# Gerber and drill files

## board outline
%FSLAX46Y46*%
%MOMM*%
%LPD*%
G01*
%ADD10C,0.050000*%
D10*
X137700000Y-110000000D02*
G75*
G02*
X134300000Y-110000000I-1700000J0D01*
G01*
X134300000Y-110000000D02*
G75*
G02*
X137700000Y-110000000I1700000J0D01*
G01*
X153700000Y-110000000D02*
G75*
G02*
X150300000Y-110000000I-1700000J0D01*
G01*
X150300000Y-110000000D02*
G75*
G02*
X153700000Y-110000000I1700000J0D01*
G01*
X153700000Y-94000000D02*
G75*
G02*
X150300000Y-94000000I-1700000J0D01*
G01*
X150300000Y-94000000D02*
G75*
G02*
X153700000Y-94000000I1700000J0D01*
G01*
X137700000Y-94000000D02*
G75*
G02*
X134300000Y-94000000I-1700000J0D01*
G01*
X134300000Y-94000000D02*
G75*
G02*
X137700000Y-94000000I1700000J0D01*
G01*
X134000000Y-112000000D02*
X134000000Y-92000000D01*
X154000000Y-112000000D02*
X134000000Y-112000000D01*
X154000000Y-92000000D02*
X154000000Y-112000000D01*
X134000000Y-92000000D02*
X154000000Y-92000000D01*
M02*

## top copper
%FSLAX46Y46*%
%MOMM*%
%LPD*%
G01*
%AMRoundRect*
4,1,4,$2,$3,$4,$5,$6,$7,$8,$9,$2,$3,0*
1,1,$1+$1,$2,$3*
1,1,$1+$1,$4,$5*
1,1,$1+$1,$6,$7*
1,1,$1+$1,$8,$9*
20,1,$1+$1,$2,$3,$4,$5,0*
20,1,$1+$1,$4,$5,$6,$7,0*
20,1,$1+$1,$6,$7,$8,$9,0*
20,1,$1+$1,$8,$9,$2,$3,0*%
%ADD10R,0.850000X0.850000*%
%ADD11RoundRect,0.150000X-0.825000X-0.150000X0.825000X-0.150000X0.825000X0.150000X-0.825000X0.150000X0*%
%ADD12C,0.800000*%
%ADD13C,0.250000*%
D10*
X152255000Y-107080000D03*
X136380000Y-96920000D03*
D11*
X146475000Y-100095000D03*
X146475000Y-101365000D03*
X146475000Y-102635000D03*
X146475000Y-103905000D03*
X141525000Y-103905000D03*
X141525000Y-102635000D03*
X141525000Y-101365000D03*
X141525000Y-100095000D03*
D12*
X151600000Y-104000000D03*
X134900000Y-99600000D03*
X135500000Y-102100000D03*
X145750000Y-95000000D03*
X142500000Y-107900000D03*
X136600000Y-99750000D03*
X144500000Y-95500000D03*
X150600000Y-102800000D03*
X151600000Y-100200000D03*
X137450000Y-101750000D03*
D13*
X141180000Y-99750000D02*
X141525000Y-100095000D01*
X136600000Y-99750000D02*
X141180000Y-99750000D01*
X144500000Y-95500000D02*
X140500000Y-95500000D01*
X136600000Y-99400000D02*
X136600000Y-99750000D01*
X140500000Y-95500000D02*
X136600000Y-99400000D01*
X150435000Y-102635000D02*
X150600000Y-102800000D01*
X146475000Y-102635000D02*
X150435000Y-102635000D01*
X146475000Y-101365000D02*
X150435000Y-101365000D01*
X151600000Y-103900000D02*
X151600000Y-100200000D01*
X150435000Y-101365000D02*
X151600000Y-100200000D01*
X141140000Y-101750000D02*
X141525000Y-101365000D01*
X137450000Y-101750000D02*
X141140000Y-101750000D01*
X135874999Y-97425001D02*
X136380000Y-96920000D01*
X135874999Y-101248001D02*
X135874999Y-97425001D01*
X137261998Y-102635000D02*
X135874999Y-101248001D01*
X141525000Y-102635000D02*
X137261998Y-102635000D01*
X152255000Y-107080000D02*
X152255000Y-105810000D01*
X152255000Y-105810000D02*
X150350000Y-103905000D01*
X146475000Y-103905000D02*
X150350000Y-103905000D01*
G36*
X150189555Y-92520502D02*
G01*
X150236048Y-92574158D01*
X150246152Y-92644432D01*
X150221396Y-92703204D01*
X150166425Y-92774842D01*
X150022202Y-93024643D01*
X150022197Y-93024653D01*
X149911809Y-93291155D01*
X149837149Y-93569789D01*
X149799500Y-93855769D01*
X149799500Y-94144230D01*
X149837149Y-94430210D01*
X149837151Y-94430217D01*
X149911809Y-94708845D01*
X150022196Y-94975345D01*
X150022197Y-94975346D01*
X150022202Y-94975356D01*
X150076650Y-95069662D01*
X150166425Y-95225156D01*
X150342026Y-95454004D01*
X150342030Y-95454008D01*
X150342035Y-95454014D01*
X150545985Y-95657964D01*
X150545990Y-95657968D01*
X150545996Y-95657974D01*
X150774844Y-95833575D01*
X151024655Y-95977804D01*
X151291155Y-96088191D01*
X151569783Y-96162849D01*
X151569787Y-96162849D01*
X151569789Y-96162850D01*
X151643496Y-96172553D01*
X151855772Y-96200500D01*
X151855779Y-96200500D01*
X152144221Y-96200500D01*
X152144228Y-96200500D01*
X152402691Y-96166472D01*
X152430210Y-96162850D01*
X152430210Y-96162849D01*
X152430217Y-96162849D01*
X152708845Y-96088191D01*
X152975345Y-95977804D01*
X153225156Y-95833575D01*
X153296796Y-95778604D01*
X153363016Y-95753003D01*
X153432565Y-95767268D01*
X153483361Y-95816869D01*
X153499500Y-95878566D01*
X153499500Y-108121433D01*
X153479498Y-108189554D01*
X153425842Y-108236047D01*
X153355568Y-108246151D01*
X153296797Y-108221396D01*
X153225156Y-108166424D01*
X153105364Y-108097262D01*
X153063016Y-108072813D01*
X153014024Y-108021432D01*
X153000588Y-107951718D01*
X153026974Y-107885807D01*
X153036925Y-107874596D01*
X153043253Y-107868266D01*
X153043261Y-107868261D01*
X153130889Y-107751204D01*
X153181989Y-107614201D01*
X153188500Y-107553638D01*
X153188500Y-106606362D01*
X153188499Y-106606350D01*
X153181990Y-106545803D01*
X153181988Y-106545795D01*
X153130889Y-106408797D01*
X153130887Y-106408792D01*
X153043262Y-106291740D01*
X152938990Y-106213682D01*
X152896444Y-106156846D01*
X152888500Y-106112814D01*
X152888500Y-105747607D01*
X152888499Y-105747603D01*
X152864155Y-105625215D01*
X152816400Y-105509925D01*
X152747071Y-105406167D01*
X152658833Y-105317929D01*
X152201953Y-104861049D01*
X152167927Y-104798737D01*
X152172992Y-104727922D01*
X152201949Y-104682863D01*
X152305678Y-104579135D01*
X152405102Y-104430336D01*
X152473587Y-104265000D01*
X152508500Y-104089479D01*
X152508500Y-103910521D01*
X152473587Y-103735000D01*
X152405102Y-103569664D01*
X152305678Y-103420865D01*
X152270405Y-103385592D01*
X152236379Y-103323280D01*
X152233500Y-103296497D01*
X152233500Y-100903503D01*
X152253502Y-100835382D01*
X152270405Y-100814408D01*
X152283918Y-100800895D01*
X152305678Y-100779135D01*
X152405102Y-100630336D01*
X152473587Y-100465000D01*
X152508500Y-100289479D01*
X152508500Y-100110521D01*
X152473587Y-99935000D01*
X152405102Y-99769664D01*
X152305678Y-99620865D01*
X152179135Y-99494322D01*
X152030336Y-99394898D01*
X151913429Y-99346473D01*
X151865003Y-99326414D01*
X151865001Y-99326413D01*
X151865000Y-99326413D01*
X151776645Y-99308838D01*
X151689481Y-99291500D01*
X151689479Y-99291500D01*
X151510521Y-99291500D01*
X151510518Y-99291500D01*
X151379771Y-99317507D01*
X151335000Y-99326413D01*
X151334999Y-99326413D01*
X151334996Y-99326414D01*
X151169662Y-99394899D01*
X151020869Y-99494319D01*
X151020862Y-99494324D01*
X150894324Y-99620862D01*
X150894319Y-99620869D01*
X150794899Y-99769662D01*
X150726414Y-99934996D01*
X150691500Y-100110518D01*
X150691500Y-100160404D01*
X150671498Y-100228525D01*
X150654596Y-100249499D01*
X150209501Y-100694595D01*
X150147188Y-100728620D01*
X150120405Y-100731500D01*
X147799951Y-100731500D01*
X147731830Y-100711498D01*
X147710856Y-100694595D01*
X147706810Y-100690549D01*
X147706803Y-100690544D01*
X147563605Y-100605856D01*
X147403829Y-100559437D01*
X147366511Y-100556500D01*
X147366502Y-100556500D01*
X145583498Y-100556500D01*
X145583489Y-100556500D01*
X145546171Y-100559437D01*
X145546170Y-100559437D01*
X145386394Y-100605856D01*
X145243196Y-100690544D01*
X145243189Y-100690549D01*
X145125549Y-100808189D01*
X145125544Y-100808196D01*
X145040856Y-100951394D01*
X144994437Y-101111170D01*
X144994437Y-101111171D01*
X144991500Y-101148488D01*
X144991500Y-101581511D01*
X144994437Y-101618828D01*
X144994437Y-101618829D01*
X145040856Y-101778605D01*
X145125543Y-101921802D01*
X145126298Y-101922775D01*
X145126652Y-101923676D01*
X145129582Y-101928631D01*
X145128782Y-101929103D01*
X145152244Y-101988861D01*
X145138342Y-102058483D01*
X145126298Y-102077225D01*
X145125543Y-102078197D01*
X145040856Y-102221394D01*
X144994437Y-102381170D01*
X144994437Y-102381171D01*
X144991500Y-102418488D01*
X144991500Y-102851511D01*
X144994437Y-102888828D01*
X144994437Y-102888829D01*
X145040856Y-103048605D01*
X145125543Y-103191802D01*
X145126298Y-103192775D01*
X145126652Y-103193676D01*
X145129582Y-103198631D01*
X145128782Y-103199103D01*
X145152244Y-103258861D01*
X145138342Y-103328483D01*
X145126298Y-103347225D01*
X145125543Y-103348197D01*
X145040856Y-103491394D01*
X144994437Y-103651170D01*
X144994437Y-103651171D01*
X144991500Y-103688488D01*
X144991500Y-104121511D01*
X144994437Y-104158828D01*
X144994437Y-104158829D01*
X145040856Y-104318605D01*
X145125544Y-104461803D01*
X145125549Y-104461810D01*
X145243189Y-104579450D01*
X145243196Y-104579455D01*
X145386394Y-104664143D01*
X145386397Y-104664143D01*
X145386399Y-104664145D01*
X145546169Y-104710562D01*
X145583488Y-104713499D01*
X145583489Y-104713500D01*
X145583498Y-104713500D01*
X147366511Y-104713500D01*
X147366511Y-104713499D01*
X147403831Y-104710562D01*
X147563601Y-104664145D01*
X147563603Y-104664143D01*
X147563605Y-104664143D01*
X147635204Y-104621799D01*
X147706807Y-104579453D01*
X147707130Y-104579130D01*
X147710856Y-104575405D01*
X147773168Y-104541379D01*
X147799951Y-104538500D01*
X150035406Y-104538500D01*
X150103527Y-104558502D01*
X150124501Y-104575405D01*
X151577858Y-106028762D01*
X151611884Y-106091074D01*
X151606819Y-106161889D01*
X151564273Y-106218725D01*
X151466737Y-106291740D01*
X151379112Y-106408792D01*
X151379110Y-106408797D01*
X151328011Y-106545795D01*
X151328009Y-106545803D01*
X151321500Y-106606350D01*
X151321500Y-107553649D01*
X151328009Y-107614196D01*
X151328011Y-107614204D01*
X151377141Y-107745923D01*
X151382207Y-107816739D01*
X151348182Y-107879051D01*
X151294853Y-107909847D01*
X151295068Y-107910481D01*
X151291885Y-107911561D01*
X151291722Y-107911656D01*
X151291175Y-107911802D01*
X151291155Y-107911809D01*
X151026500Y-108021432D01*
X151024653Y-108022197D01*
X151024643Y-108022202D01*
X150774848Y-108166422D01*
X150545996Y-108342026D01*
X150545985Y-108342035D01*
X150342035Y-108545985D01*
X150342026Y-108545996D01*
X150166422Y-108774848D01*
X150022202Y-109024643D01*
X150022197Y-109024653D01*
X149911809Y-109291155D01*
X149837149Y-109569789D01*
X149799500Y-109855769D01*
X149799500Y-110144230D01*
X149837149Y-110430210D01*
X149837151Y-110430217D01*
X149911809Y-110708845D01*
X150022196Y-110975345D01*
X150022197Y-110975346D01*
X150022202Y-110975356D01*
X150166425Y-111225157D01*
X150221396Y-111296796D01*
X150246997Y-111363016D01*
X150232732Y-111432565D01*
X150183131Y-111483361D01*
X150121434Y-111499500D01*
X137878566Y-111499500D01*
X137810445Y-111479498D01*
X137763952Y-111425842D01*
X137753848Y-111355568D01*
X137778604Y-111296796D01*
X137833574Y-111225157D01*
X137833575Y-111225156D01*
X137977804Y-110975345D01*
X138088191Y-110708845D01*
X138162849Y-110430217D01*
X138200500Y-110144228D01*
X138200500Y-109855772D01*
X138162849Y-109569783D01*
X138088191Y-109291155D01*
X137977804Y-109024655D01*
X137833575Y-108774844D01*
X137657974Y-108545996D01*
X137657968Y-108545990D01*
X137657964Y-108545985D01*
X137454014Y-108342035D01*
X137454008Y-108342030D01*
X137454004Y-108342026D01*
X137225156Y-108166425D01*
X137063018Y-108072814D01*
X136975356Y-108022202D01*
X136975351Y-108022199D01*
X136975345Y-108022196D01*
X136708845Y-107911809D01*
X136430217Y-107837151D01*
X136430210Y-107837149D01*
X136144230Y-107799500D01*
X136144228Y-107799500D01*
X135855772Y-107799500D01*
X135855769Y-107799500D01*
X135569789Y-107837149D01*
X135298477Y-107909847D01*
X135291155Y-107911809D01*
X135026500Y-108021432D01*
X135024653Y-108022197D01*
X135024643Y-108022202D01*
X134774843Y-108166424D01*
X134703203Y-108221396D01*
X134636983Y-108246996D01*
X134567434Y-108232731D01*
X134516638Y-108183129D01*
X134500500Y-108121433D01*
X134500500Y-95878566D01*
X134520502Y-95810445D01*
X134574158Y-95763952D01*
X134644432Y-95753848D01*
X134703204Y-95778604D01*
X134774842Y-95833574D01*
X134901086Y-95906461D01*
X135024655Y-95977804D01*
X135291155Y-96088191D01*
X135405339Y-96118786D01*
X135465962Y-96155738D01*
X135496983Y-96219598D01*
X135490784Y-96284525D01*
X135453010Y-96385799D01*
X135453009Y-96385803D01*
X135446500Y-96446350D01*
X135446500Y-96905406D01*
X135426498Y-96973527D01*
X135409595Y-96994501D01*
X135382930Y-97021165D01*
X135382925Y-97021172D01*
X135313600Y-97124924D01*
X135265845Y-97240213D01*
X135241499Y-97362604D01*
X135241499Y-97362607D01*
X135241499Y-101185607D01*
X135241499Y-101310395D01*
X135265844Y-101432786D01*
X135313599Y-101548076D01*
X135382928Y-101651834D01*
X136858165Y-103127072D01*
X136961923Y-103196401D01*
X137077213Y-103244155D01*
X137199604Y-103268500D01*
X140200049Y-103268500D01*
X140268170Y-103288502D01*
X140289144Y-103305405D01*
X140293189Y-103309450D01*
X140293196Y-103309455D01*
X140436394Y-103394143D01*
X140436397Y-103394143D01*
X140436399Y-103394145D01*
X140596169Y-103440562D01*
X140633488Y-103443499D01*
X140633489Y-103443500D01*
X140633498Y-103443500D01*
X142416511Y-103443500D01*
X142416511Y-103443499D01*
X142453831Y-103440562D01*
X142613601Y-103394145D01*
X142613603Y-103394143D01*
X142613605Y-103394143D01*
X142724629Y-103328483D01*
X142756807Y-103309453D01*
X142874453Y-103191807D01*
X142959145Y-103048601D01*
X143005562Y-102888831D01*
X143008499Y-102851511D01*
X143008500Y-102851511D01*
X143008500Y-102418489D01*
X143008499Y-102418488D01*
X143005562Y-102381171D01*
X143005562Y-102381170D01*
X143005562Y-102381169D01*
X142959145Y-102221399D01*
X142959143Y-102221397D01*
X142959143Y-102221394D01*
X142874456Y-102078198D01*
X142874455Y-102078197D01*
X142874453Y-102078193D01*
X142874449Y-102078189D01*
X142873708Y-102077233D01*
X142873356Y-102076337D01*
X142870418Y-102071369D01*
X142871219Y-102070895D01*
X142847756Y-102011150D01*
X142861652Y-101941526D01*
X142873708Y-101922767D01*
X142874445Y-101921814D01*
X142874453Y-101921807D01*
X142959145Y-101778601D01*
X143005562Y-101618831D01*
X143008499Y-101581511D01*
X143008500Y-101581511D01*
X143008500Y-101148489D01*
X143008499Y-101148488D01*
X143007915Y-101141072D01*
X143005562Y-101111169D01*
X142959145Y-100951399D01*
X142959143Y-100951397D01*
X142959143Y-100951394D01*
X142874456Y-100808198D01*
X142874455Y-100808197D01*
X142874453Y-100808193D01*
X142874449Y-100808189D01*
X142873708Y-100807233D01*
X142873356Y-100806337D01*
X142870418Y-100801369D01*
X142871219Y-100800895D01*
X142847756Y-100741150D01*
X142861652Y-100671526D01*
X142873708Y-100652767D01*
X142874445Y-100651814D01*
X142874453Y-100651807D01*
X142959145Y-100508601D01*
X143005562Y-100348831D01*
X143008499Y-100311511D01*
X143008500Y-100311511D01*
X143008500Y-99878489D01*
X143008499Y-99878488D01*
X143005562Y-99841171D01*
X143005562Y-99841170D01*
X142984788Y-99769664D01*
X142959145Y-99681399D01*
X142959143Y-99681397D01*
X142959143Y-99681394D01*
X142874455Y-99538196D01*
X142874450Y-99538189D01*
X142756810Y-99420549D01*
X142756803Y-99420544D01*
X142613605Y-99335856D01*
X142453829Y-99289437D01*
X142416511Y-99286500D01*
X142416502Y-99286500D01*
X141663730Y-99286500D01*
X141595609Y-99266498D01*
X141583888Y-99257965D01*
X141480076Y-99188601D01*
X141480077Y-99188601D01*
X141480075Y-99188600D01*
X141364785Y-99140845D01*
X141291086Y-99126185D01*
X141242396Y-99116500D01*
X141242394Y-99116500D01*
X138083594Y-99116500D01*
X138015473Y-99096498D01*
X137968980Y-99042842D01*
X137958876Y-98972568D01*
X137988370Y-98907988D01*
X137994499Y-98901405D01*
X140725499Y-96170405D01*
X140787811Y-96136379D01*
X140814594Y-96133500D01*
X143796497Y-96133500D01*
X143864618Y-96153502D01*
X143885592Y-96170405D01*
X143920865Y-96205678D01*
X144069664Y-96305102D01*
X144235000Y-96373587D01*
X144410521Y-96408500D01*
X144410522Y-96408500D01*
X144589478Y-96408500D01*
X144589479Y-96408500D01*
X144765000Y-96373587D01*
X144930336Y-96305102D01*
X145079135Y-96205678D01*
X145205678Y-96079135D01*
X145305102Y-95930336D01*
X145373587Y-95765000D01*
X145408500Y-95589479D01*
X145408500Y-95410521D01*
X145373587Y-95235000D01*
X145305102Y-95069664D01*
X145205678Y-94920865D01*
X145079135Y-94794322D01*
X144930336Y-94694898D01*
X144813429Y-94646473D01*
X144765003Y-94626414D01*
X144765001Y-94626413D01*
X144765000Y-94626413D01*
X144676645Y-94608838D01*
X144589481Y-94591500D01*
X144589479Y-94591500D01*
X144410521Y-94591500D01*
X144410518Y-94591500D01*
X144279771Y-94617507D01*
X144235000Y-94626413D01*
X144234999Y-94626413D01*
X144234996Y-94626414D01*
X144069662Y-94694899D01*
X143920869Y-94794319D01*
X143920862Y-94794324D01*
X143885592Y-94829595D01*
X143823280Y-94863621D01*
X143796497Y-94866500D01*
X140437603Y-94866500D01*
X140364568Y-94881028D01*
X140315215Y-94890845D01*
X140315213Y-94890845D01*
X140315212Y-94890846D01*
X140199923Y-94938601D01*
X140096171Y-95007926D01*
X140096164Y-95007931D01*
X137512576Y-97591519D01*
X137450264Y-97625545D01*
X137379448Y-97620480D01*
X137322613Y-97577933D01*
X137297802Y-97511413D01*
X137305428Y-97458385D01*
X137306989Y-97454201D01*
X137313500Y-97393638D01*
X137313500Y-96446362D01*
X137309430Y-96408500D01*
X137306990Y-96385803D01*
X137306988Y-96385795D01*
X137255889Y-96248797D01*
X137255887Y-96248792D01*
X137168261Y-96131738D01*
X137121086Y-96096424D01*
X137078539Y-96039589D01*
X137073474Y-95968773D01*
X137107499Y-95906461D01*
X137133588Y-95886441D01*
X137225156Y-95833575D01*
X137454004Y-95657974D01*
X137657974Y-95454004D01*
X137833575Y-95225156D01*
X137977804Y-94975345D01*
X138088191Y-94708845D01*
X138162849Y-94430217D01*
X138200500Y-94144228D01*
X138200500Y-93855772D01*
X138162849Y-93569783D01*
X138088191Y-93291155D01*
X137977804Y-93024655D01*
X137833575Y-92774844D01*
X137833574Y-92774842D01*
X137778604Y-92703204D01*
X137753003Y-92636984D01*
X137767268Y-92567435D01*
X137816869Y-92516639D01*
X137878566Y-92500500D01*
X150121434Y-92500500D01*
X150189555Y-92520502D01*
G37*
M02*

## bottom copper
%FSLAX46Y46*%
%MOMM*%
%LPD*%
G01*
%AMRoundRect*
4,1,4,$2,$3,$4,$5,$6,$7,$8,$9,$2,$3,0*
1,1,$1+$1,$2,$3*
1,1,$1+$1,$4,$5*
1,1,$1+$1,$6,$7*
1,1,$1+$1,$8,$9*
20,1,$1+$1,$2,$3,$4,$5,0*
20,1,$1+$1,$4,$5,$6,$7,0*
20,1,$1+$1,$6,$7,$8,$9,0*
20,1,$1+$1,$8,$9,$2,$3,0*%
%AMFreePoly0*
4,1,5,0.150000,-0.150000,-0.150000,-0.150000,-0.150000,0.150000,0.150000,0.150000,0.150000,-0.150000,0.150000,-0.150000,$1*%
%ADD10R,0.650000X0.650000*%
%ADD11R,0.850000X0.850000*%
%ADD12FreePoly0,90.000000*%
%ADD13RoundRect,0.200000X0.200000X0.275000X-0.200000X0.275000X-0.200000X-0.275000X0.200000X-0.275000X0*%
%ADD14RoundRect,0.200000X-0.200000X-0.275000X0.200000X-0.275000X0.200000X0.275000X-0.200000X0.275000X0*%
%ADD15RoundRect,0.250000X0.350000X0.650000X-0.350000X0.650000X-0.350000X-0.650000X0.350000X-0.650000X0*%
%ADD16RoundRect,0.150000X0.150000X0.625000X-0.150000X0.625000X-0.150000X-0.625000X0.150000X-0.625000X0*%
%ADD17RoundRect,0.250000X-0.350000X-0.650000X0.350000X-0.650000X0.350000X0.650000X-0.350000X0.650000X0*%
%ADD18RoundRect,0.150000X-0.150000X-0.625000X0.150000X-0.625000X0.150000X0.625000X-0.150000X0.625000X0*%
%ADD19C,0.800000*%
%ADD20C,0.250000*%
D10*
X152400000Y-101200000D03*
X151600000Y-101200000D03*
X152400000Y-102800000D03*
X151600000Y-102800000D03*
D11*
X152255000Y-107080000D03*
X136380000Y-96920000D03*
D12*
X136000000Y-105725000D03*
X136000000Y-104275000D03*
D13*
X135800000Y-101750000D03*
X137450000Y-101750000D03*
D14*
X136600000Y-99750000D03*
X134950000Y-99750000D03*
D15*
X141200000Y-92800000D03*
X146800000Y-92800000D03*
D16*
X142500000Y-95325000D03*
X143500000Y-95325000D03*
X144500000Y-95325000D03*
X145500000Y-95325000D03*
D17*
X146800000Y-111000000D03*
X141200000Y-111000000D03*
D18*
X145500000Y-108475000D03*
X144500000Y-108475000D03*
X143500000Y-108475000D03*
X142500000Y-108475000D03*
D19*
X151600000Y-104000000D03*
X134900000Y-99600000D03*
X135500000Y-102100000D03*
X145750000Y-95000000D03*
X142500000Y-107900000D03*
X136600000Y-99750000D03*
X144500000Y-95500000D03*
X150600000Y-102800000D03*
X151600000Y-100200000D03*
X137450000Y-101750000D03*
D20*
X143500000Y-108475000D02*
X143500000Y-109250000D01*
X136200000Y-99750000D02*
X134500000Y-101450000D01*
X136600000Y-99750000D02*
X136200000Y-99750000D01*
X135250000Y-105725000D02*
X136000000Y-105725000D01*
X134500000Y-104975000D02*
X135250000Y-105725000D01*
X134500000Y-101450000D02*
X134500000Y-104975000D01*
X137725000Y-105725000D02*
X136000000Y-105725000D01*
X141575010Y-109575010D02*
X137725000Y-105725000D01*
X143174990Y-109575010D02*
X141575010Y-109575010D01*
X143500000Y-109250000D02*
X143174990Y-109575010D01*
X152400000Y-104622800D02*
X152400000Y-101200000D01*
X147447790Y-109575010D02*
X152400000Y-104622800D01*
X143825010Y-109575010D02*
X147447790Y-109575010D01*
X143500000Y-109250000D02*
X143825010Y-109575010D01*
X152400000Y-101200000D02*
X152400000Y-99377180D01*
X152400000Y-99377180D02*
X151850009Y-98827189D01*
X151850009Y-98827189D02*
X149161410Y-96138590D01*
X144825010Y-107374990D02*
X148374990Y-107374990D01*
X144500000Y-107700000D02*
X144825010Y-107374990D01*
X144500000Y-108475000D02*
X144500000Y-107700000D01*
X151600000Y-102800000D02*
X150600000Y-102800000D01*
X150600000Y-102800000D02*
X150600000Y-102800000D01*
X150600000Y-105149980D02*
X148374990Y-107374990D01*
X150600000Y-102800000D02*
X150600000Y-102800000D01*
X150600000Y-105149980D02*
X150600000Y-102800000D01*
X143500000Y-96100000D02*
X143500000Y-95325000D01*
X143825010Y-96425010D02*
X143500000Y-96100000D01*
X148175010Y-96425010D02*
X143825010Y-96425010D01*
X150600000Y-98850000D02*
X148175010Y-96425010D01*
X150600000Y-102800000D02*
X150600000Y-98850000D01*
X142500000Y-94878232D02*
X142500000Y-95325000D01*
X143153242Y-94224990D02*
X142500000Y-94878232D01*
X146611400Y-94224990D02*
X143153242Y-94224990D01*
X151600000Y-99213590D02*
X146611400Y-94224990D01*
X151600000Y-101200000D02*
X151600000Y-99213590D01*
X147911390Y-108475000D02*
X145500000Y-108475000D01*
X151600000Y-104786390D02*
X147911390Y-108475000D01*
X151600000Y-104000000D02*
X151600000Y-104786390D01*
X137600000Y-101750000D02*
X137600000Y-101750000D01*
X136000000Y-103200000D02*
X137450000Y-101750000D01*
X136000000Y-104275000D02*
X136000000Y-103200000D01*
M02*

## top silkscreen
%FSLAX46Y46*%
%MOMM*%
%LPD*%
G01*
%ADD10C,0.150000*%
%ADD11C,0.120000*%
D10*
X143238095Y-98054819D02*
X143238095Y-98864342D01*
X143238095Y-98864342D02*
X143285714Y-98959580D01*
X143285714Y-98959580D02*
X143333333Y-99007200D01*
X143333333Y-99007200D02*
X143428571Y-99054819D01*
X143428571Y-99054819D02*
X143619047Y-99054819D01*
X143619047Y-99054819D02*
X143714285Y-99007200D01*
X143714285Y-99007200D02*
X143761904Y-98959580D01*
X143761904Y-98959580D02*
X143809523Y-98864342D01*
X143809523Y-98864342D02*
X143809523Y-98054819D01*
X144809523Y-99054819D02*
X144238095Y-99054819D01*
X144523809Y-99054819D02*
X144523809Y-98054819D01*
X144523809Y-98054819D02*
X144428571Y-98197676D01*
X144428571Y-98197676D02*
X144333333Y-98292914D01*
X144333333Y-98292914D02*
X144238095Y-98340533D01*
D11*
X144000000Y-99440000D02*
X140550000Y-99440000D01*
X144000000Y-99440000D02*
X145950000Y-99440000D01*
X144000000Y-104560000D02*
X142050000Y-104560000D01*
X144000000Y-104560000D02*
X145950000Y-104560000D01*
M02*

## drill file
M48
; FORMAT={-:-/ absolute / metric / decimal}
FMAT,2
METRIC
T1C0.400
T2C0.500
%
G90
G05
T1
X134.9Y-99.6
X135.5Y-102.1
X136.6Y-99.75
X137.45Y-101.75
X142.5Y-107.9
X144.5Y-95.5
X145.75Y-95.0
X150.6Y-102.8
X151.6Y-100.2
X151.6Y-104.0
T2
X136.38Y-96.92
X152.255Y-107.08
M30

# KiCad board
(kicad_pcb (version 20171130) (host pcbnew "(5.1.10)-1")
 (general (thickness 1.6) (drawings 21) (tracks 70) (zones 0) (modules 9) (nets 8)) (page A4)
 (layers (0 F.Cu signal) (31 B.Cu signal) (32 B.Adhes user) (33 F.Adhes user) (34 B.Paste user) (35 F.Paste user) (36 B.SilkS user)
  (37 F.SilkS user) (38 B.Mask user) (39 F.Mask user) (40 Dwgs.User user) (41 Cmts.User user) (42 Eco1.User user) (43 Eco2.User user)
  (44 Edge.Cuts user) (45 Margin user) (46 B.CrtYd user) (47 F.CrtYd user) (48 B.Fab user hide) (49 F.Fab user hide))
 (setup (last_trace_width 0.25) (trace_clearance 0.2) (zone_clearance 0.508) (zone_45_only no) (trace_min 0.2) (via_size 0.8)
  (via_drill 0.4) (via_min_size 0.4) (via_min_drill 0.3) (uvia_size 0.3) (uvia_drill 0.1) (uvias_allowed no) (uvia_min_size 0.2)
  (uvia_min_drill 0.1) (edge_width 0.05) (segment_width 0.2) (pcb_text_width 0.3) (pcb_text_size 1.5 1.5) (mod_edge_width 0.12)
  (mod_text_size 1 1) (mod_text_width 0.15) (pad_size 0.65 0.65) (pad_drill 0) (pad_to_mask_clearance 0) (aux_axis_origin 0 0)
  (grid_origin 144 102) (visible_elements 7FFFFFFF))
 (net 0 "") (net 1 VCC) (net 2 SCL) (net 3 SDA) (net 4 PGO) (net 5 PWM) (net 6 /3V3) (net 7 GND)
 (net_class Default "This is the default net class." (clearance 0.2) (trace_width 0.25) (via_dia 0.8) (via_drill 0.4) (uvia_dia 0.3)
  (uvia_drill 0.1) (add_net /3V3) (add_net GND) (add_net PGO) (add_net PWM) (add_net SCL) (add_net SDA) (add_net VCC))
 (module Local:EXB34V (layer B.Cu) (at 152 102)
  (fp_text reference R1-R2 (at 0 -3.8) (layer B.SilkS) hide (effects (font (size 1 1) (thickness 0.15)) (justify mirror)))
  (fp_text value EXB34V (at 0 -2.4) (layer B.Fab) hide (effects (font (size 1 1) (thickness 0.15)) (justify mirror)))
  (pad 4 smd rect (at 0.4 -0.8) (size 0.65 0.65) (layers B.Cu B.Paste B.Mask) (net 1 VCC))
  (pad 3 smd rect (at -0.4 -0.8) (size 0.65 0.65) (layers B.Cu B.Paste B.Mask) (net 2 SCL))
  (pad 2 smd rect (at 0.4 0.8) (size 0.65 0.65) (layers B.Cu B.Paste B.Mask) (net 1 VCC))
  (pad 1 smd rect (at -0.4 0.8) (size 0.65 0.65) (layers B.Cu B.Paste B.Mask) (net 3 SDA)))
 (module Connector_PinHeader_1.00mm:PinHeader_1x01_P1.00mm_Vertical (layer B.Cu) (at 152.255 107.08)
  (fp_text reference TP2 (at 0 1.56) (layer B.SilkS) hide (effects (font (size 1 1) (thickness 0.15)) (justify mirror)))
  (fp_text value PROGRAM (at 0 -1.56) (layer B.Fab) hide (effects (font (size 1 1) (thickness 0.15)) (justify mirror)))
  (pad 1 thru_hole rect (at 0 0) (size 0.85 0.85) (drill 0.5) (layers *.Cu *.Mask) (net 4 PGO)))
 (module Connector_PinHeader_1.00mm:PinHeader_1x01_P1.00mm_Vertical (layer B.Cu) (at 136.38 96.92)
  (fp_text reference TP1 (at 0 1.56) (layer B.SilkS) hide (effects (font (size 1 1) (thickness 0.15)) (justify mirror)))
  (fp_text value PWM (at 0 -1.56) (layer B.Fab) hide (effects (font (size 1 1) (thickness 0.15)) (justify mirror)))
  (pad 1 thru_hole rect (at 0 0) (size 0.85 0.85) (drill 0.5) (layers *.Cu *.Mask) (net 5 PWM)))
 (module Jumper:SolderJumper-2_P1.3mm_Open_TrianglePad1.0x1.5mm (layer B.Cu) (at 136 105 90)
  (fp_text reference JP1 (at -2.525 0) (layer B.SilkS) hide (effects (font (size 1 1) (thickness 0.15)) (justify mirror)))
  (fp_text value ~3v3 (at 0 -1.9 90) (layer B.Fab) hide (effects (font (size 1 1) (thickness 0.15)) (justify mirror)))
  (pad 1 smd custom (at -0.725 0 90) (size 0.3 0.3) (layers B.Cu B.Mask) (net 1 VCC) (zone_connect 2)
   (options (clearance outline) (anchor rect)) (primitives))
  (pad 2 smd custom (at 0.725 0 90) (size 0.3 0.3) (layers B.Cu B.Mask) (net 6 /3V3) (zone_connect 2)
   (options (clearance outline) (anchor rect)) (primitives)))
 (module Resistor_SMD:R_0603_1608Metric (layer B.Cu) (at 136.625 101.75 180)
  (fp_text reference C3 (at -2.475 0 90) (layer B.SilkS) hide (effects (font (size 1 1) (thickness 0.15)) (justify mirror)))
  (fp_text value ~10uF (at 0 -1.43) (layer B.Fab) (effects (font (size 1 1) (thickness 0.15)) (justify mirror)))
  (pad 2 smd roundrect (at 0.825 0 180) (size 0.8 0.95) (layers B.Cu B.Paste B.Mask) (roundrect_rratio 0.25) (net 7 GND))
  (pad 1 smd roundrect (at -0.825 0 180) (size 0.8 0.95) (layers B.Cu B.Paste B.Mask) (roundrect_rratio 0.25) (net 6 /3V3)))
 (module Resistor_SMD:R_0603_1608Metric (layer B.Cu) (at 135.775 99.75)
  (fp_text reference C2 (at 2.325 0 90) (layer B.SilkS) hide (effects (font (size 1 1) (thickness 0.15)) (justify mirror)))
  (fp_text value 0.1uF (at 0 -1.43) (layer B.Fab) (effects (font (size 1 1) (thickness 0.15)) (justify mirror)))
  (pad 2 smd roundrect (at 0.825 0) (size 0.8 0.95) (layers B.Cu B.Paste B.Mask) (roundrect_rratio 0.25) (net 1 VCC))
  (pad 1 smd roundrect (at -0.825 0) (size 0.8 0.95) (layers B.Cu B.Paste B.Mask) (roundrect_rratio 0.25) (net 7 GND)))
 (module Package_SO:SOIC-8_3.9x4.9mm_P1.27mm (layer F.Cu) (at 144 102)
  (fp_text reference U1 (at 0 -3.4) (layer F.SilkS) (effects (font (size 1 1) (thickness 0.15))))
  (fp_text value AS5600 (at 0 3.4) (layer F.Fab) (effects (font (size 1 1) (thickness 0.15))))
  (fp_line (start 0 -2.56) (end -3.45 -2.56) (layer F.SilkS) (width 0.12))
  (fp_line (start 0 -2.56) (end 1.95 -2.56) (layer F.SilkS) (width 0.12))
  (fp_line (start 0 2.56) (end -1.95 2.56) (layer F.SilkS) (width 0.12))
  (fp_line (start 0 2.56) (end 1.95 2.56) (layer F.SilkS) (width 0.12))
  (pad 8 smd roundrect (at 2.475 -1.905) (size 1.95 0.6) (layers F.Cu F.Paste F.Mask) (roundrect_rratio 0.25) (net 7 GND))
  (pad 7 smd roundrect (at 2.475 -0.635) (size 1.95 0.6) (layers F.Cu F.Paste F.Mask) (roundrect_rratio 0.25) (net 2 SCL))
  (pad 6 smd roundrect (at 2.475 0.635) (size 1.95 0.6) (layers F.Cu F.Paste F.Mask) (roundrect_rratio 0.25) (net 3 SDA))
  (pad 5 smd roundrect (at 2.475 1.905) (size 1.95 0.6) (layers F.Cu F.Paste F.Mask) (roundrect_rratio 0.25) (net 4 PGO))
  (pad 4 smd roundrect (at -2.475 1.905) (size 1.95 0.6) (layers F.Cu F.Paste F.Mask) (roundrect_rratio 0.25) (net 7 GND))
  (pad 3 smd roundrect (at -2.475 0.635) (size 1.95 0.6) (layers F.Cu F.Paste F.Mask) (roundrect_rratio 0.25) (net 5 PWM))
  (pad 2 smd roundrect (at -2.475 -0.635) (size 1.95 0.6) (layers F.Cu F.Paste F.Mask) (roundrect_rratio 0.25) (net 6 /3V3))
  (pad 1 smd roundrect (at -2.475 -1.905) (size 1.95 0.6) (layers F.Cu F.Paste F.Mask) (roundrect_rratio 0.25) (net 1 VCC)))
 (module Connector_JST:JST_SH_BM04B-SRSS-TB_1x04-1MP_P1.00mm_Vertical (layer B.Cu) (at 144 94 180)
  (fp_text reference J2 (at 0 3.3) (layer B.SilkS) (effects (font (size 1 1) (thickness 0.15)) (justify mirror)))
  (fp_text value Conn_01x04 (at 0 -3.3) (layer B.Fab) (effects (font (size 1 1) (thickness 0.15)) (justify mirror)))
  (pad MP smd roundrect (at 2.8 1.2 180) (size 1.2 1.8) (layers B.Cu B.Paste B.Mask) (roundrect_rratio 0.208333))
  (pad MP smd roundrect (at -2.8 1.2 180) (size 1.2 1.8) (layers B.Cu B.Paste B.Mask) (roundrect_rratio 0.208333))
  (pad 4 smd roundrect (at 1.5 -1.325 180) (size 0.6 1.55) (layers B.Cu B.Paste B.Mask) (roundrect_rratio 0.25) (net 2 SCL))
  (pad 3 smd roundrect (at 0.5 -1.325 180) (size 0.6 1.55) (layers B.Cu B.Paste B.Mask) (roundrect_rratio 0.25) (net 3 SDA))
  (pad 2 smd roundrect (at -0.5 -1.325 180) (size 0.6 1.55) (layers B.Cu B.Paste B.Mask) (roundrect_rratio 0.25) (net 1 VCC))
  (pad 1 smd roundrect (at -1.5 -1.325 180) (size 0.6 1.55) (layers B.Cu B.Paste B.Mask) (roundrect_rratio 0.25) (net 7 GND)))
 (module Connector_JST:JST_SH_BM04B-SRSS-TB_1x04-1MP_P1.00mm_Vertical (layer B.Cu) (at 144 109.8)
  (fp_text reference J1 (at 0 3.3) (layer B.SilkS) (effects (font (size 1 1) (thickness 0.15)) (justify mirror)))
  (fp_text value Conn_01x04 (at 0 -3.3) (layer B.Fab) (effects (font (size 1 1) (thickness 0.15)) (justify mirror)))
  (pad MP smd roundrect (at 2.8 1.2) (size 1.2 1.8) (layers B.Cu B.Paste B.Mask) (roundrect_rratio 0.208333))
  (pad MP smd roundrect (at -2.8 1.2) (size 1.2 1.8) (layers B.Cu B.Paste B.Mask) (roundrect_rratio 0.208333))
  (pad 4 smd roundrect (at 1.5 -1.325) (size 0.6 1.55) (layers B.Cu B.Paste B.Mask) (roundrect_rratio 0.25) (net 2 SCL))
  (pad 3 smd roundrect (at 0.5 -1.325) (size 0.6 1.55) (layers B.Cu B.Paste B.Mask) (roundrect_rratio 0.25) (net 3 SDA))
  (pad 2 smd roundrect (at -0.5 -1.325) (size 0.6 1.55) (layers B.Cu B.Paste B.Mask) (roundrect_rratio 0.25) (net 1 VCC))
  (pad 1 smd roundrect (at -1.5 -1.325) (size 0.6 1.55) (layers B.Cu B.Paste B.Mask) (roundrect_rratio 0.25) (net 7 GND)))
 (gr_circle (center 136 110) (end 137.7 110) (layer Edge.Cuts) (width 0.05))
 (gr_circle (center 152 110) (end 153.7 110) (layer Edge.Cuts) (width 0.05))
 (gr_circle (center 152 94) (end 153.7 94) (layer Edge.Cuts) (width 0.05))
 (gr_circle (center 136 94) (end 137.7 94) (layer Edge.Cuts) (width 0.05))
 (gr_line (start 134 112) (end 134 92) (layer Edge.Cuts) (width 0.05))
 (gr_line (start 154 112) (end 134 112) (layer Edge.Cuts) (width 0.05))
 (gr_line (start 154 92) (end 154 112) (layer Edge.Cuts) (width 0.05))
 (gr_line (start 134 92) (end 154 92) (layer Edge.Cuts) (width 0.05))
 (via (at 151.6 104) (size 0.8) (drill 0.4) (layers F.Cu B.Cu) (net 2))
 (via (at 134.9 99.6) (size 0.8) (drill 0.4) (layers F.Cu B.Cu) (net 7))
 (via (at 135.5 102.1) (size 0.8) (drill 0.4) (layers F.Cu B.Cu) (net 7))
 (via (at 145.75 95) (size 0.8) (drill 0.4) (layers F.Cu B.Cu) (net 7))
 (via (at 142.5 107.9) (size 0.8) (drill 0.4) (layers F.Cu B.Cu) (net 7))
 (segment (start 143.5 108.475) (end 143.5 109.25) (width 0.25) (layer B.Cu) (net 1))
 (via (at 136.6 99.75) (size 0.8) (drill 0.4) (layers F.Cu B.Cu) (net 1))
 (via (at 144.5 95.5) (size 0.8) (drill 0.4) (layers F.Cu B.Cu) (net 1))
 (segment (start 141.18 99.75) (end 141.525 100.095) (width 0.25) (layer F.Cu) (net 1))
 (segment (start 136.6 99.75) (end 141.18 99.75) (width 0.25) (layer F.Cu) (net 1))
 (segment (start 136.2 99.75) (end 134.5 101.45) (width 0.25) (layer B.Cu) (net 1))
 (segment (start 136.6 99.75) (end 136.2 99.75) (width 0.25) (layer B.Cu) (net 1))
 (segment (start 135.25 105.725) (end 136 105.725) (width 0.25) (layer B.Cu) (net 1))
 (segment (start 134.5 104.975) (end 135.25 105.725) (width 0.25) (layer B.Cu) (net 1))
 (segment (start 134.5 101.45) (end 134.5 104.975) (width 0.25) (layer B.Cu) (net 1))
 (segment (start 144.5 95.5) (end 140.5 95.5) (width 0.25) (layer F.Cu) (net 1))
 (segment (start 136.6 99.4) (end 136.6 99.75) (width 0.25) (layer F.Cu) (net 1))
 (segment (start 140.5 95.5) (end 136.6 99.4) (width 0.25) (layer F.Cu) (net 1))
 (segment (start 137.725 105.725) (end 136 105.725) (width 0.25) (layer B.Cu) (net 1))
 (segment (start 141.57501 109.57501) (end 137.725 105.725) (width 0.25) (layer B.Cu) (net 1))
 (segment (start 143.17499 109.57501) (end 141.57501 109.57501) (width 0.25) (layer B.Cu) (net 1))
 (segment (start 143.5 109.25) (end 143.17499 109.57501) (width 0.25) (layer B.Cu) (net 1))
 (segment (start 152.4 104.6228) (end 152.4 101.2) (width 0.25) (layer B.Cu) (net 1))
 (segment (start 147.44779 109.57501) (end 152.4 104.6228) (width 0.25) (layer B.Cu) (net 1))
 (segment (start 143.82501 109.57501) (end 147.44779 109.57501) (width 0.25) (layer B.Cu) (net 1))
 (segment (start 143.5 109.25) (end 143.82501 109.57501) (width 0.25) (layer B.Cu) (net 1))
 (segment (start 152.4 101.2) (end 152.4 99.37718) (width 0.25) (layer B.Cu) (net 1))
 (segment (start 152.4 99.37718) (end 151.850009 98.827189) (width 0.25) (layer B.Cu) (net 1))
 (segment (start 151.850009 98.827189) (end 149.16141 96.13859) (width 0.25) (layer B.Cu) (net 1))
 (segment (start 144.82501 107.37499) (end 148.37499 107.37499) (width 0.25) (layer B.Cu) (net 3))
 (segment (start 144.5 107.7) (end 144.82501 107.37499) (width 0.25) (layer B.Cu) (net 3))
 (segment (start 144.5 108.475) (end 144.5 107.7) (width 0.25) (layer B.Cu) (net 3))
 (segment (start 151.6 102.8) (end 150.6 102.8) (width 0.25) (layer B.Cu) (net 3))
 (segment (start 150.6 102.8) (end 150.6 102.8) (width 0.25) (layer B.Cu) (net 3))
 (segment (start 150.6 105.14998) (end 148.37499 107.37499) (width 0.25) (layer B.Cu) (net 3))
 (segment (start 150.6 102.8) (end 150.6 102.8) (width 0.25) (layer B.Cu) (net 3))
 (via (at 150.6 102.8) (size 0.8) (drill 0.4) (layers F.Cu B.Cu) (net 3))
 (segment (start 150.435 102.635) (end 150.6 102.8) (width 0.25) (layer F.Cu) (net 3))
 (segment (start 146.475 102.635) (end 150.435 102.635) (width 0.25) (layer F.Cu) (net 3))
 (segment (start 150.6 105.14998) (end 150.6 102.8) (width 0.25) (layer B.Cu) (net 3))
 (segment (start 143.5 96.1) (end 143.5 95.325) (width 0.25) (layer B.Cu) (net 3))
 (segment (start 143.82501 96.42501) (end 143.5 96.1) (width 0.25) (layer B.Cu) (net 3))
 (segment (start 148.17501 96.42501) (end 143.82501 96.42501) (width 0.25) (layer B.Cu) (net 3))
 (segment (start 150.6 98.85) (end 148.17501 96.42501) (width 0.25) (layer B.Cu) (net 3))
 (segment (start 150.6 102.8) (end 150.6 98.85) (width 0.25) (layer B.Cu) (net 3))
 (via (at 151.6 100.2) (size 0.8) (drill 0.4) (layers F.Cu B.Cu) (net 2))
 (segment (start 142.5 94.878232) (end 142.5 95.325) (width 0.25) (layer B.Cu) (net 2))
 (segment (start 143.153242 94.22499) (end 142.5 94.878232) (width 0.25) (layer B.Cu) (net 2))
 (segment (start 146.6114 94.22499) (end 143.153242 94.22499) (width 0.25) (layer B.Cu) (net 2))
 (segment (start 151.6 99.21359) (end 146.6114 94.22499) (width 0.25) (layer B.Cu) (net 2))
 (segment (start 151.6 101.2) (end 151.6 99.21359) (width 0.25) (layer B.Cu) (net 2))
 (segment (start 146.475 101.365) (end 150.435 101.365) (width 0.25) (layer F.Cu) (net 2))
 (segment (start 151.6 103.9) (end 151.6 100.2) (width 0.25) (layer F.Cu) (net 2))
 (segment (start 147.91139 108.475) (end 145.5 108.475) (width 0.25) (layer B.Cu) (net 2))
 (segment (start 151.6 104.78639) (end 147.91139 108.475) (width 0.25) (layer B.Cu) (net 2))
 (segment (start 151.6 104) (end 151.6 104.78639) (width 0.25) (layer B.Cu) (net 2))
 (segment (start 150.435 101.365) (end 151.6 100.2) (width 0.25) (layer F.Cu) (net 2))
 (segment (start 137.6 101.75) (end 137.6 101.75) (width 0.25) (layer B.Cu) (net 6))
 (via (at 137.45 101.75) (size 0.8) (drill 0.4) (layers F.Cu B.Cu) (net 6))
 (segment (start 141.14 101.75) (end 141.525 101.365) (width 0.25) (layer F.Cu) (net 6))
 (segment (start 137.45 101.75) (end 141.14 101.75) (width 0.25) (layer F.Cu) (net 6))
 (segment (start 136 103.2) (end 137.45 101.75) (width 0.25) (layer B.Cu) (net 6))
 (segment (start 136 104.275) (end 136 103.2) (width 0.25) (layer B.Cu) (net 6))
 (segment (start 135.874999 97.425001) (end 136.38 96.92) (width 0.25) (layer F.Cu) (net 5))
 (segment (start 135.874999 101.248001) (end 135.874999 97.425001) (width 0.25) (layer F.Cu) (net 5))
 (segment (start 137.261998 102.635) (end 135.874999 101.248001) (width 0.25) (layer F.Cu) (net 5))
 (segment (start 141.525 102.635) (end 137.261998 102.635) (width 0.25) (layer F.Cu) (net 5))
 (segment (start 152.255 107.08) (end 152.255 105.81) (width 0.25) (layer F.Cu) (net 4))
 (segment (start 152.255 105.81) (end 150.35 103.905) (width 0.25) (layer F.Cu) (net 4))
 (segment (start 146.475 103.905) (end 150.35 103.905) (width 0.25) (layer F.Cu) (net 4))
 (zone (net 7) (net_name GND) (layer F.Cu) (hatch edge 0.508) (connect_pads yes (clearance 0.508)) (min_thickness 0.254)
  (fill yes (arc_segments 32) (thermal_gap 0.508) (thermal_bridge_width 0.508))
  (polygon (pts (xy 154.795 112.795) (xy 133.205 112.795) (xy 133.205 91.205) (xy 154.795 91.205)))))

